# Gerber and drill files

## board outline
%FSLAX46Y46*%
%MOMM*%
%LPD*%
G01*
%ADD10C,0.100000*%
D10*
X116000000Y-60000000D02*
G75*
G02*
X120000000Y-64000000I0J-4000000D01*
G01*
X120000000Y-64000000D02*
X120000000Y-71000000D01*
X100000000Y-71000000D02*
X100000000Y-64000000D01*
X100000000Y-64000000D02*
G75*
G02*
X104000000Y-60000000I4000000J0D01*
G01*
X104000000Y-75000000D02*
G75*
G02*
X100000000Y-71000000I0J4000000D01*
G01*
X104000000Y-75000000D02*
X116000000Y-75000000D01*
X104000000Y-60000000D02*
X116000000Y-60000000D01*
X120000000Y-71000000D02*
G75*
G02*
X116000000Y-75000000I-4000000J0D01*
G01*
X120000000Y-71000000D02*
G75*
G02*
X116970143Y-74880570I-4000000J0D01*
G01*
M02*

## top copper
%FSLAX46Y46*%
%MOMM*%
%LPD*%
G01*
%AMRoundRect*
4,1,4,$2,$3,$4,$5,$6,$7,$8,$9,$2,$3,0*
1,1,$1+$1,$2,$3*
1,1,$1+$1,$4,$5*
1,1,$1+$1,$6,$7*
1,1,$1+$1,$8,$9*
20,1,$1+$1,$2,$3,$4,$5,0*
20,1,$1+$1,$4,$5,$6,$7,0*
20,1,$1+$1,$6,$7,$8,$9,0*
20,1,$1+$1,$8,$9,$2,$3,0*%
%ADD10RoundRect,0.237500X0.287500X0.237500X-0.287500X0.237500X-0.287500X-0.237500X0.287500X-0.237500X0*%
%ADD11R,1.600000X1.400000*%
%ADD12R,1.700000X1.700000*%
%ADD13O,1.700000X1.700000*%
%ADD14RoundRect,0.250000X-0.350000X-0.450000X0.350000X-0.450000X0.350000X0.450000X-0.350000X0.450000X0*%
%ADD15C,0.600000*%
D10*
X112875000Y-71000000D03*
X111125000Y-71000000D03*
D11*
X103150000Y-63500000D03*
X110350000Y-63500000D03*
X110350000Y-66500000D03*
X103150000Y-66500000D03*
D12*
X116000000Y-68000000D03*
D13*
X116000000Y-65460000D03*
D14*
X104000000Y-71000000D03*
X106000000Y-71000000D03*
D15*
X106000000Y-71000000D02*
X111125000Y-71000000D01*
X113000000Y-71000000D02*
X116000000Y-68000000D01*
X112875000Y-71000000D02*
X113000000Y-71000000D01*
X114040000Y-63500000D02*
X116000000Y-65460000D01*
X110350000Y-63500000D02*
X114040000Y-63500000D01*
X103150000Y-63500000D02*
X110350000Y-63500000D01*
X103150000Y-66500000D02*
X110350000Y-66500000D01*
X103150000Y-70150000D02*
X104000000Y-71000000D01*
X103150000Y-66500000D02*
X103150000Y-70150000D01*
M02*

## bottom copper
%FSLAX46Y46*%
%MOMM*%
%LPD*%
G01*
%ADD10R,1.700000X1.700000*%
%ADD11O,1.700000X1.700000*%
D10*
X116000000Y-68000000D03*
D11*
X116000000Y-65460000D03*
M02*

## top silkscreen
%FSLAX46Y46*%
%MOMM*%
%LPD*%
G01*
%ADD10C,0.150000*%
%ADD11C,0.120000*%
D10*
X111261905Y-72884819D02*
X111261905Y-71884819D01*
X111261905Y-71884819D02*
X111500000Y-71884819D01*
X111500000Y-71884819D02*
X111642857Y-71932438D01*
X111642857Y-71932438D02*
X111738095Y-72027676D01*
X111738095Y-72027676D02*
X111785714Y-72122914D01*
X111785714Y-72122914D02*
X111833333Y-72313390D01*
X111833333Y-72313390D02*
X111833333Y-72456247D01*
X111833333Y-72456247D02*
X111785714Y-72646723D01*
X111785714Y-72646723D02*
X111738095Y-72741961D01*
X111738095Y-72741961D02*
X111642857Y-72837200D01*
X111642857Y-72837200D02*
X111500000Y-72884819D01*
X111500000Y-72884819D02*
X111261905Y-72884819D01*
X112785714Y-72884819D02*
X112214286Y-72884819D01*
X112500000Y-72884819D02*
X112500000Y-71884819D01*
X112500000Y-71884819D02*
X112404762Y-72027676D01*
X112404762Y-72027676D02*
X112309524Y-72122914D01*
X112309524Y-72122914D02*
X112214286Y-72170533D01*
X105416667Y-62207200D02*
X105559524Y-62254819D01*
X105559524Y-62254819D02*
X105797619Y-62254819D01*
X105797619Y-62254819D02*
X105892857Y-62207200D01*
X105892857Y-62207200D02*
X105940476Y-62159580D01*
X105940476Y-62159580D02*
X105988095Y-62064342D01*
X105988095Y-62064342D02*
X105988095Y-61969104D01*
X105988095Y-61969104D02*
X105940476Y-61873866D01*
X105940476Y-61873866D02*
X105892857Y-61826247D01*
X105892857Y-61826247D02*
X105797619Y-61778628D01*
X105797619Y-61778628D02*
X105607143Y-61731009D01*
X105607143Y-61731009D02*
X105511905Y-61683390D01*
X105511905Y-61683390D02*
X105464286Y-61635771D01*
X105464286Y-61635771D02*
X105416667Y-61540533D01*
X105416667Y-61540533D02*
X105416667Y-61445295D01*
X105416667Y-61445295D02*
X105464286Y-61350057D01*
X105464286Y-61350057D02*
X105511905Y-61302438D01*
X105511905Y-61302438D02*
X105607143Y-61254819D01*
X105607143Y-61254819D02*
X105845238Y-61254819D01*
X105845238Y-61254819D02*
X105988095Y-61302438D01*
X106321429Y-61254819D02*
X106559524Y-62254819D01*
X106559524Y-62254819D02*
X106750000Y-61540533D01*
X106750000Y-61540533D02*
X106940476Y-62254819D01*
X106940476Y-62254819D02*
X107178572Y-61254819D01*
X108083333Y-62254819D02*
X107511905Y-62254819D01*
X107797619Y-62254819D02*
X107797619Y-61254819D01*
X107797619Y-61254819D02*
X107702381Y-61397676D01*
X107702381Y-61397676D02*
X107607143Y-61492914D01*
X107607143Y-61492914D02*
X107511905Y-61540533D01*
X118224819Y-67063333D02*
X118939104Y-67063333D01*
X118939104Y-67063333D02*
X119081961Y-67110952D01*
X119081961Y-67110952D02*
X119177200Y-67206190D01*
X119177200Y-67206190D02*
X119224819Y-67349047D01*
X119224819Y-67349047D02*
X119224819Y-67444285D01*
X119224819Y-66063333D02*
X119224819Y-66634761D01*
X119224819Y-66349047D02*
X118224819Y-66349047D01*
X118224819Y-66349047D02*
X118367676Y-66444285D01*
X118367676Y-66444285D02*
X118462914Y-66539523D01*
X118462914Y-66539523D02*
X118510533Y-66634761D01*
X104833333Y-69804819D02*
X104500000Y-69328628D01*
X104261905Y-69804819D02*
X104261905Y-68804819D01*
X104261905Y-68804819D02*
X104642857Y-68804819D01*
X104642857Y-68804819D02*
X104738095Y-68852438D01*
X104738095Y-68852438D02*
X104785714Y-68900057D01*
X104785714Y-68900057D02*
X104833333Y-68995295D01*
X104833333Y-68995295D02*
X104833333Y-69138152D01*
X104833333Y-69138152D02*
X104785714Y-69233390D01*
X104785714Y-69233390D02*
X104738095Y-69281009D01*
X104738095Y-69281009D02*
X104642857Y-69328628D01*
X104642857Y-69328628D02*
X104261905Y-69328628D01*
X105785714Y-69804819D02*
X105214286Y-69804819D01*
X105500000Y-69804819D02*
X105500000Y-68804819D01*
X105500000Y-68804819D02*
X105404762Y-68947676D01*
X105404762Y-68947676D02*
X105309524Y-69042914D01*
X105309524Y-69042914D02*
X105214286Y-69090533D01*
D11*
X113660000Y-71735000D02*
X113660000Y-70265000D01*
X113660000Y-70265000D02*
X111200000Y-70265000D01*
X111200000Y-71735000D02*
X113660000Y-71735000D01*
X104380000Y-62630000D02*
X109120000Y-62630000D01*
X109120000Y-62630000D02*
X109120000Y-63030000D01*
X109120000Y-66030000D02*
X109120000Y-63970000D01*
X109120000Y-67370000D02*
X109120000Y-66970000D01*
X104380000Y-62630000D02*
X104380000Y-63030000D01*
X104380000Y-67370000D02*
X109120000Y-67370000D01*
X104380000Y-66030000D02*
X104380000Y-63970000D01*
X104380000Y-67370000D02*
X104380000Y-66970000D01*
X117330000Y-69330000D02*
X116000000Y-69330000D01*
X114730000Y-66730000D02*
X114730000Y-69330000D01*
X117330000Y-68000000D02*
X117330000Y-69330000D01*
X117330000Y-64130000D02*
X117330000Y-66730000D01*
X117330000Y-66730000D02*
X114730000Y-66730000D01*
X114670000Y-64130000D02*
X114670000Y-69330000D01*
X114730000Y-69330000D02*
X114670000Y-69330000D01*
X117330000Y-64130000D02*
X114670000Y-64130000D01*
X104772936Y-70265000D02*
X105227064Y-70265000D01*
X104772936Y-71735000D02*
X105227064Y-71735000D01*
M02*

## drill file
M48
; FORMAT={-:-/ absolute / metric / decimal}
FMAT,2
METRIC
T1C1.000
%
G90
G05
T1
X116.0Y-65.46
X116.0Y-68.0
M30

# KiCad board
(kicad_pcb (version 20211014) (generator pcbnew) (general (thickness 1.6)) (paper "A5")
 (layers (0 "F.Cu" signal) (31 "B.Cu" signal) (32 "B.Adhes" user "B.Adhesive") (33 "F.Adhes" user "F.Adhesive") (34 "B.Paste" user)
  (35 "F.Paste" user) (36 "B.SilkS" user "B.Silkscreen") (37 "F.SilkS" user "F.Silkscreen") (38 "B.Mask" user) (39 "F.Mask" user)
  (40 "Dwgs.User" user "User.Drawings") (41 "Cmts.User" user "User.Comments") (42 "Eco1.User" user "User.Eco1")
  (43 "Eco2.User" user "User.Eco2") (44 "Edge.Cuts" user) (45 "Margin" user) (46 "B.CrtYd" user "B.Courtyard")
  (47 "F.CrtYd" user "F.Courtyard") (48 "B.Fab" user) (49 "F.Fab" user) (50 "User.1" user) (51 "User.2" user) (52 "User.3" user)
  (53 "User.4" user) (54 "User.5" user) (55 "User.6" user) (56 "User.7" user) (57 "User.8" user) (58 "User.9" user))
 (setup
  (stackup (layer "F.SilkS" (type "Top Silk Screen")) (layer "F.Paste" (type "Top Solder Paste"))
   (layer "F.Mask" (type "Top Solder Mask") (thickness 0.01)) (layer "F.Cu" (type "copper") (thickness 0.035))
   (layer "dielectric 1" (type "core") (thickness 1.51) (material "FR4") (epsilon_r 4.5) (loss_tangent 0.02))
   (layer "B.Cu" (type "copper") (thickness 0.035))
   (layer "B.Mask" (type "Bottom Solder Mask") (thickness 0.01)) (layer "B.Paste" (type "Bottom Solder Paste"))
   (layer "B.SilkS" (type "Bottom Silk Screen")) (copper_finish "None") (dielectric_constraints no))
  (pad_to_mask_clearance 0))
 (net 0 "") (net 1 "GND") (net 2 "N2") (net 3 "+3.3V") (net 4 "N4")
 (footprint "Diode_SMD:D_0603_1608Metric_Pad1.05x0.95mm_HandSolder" (layer "F.Cu") (at 112 71 180)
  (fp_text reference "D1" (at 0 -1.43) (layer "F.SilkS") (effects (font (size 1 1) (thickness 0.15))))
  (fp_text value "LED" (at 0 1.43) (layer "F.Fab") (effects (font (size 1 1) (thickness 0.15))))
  (fp_line (start -1.66 -0.735) (end -1.66 0.735) (layer "F.SilkS") (width 0.12))
  (fp_line (start -1.66 0.735) (end 0.8 0.735) (layer "F.SilkS") (width 0.12))
  (fp_line (start 0.8 -0.735) (end -1.66 -0.735) (layer "F.SilkS") (width 0.12))
  (pad "1" smd roundrect (at -0.875 0 180) (size 1.05 0.95) (layers "F.Cu" "F.Paste" "F.Mask") (roundrect_rratio 0.25) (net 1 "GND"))
  (pad "2" smd roundrect (at 0.875 0 180) (size 1.05 0.95) (layers "F.Cu" "F.Paste" "F.Mask") (roundrect_rratio 0.25) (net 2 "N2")))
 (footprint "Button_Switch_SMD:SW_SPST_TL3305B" (layer "F.Cu") (at 106.75 65)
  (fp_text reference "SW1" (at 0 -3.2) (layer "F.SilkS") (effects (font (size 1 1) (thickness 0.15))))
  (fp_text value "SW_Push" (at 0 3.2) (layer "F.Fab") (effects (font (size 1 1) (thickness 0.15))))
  (fp_line (start -2.37 -2.37) (end 2.37 -2.37) (layer "F.SilkS") (width 0.12))
  (fp_line (start 2.37 -2.37) (end 2.37 -1.97) (layer "F.SilkS") (width 0.12))
  (fp_line (start 2.37 1.03) (end 2.37 -1.03) (layer "F.SilkS") (width 0.12))
  (fp_line (start 2.37 2.37) (end 2.37 1.97) (layer "F.SilkS") (width 0.12))
  (fp_line (start -2.37 -2.37) (end -2.37 -1.97) (layer "F.SilkS") (width 0.12))
  (fp_line (start -2.37 2.37) (end 2.37 2.37) (layer "F.SilkS") (width 0.12))
  (fp_line (start -2.37 1.03) (end -2.37 -1.03) (layer "F.SilkS") (width 0.12))
  (fp_line (start -2.37 2.37) (end -2.37 1.97) (layer "F.SilkS") (width 0.12))
  (pad "1" smd rect (at -3.6 -1.5) (size 1.6 1.4) (layers "F.Cu" "F.Paste" "F.Mask") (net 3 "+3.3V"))
  (pad "1" smd rect (at 3.6 -1.5) (size 1.6 1.4) (layers "F.Cu" "F.Paste" "F.Mask") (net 3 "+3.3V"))
  (pad "2" smd rect (at 3.6 1.5) (size 1.6 1.4) (layers "F.Cu" "F.Paste" "F.Mask") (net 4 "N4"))
  (pad "2" smd rect (at -3.6 1.5) (size 1.6 1.4) (layers "F.Cu" "F.Paste" "F.Mask") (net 4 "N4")))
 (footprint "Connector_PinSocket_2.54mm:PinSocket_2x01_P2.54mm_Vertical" (layer "F.Cu") (at 116 68 -90)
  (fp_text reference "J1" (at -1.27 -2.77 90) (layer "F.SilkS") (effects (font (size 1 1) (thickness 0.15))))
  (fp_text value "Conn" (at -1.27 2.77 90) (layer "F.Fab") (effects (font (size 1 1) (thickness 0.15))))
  (fp_line (start 1.33 -1.33) (end 1.33 0) (layer "F.SilkS") (width 0.12))
  (fp_line (start -1.27 1.27) (end 1.33 1.27) (layer "F.SilkS") (width 0.12))
  (fp_line (start 0 -1.33) (end 1.33 -1.33) (layer "F.SilkS") (width 0.12))
  (fp_line (start -3.87 -1.33) (end -1.27 -1.33) (layer "F.SilkS") (width 0.12))
  (fp_line (start -1.27 -1.33) (end -1.27 1.27) (layer "F.SilkS") (width 0.12))
  (fp_line (start -3.87 1.33) (end 1.33 1.33) (layer "F.SilkS") (width 0.12))
  (fp_line (start 1.33 1.27) (end 1.33 1.33) (layer "F.SilkS") (width 0.12))
  (fp_line (start -3.87 -1.33) (end -3.87 1.33) (layer "F.SilkS") (width 0.12))
  (pad "1" thru_hole rect (at 0 0 270) (size 1.7 1.7) (drill 1) (layers *.Cu *.Mask) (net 1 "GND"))
  (pad "2" thru_hole oval (at -2.54 0 270) (size 1.7 1.7) (drill 1) (layers *.Cu *.Mask) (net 3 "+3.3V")))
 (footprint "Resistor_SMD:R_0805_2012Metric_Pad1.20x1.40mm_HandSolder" (layer "F.Cu") (at 105 71)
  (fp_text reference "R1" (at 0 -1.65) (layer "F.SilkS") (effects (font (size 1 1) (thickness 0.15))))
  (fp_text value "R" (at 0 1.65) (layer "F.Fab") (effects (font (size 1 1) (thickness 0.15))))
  (fp_line (start -0.227064 -0.735) (end 0.227064 -0.735) (layer "F.SilkS") (width 0.12))
  (fp_line (start -0.227064 0.735) (end 0.227064 0.735) (layer "F.SilkS") (width 0.12))
  (pad "1" smd roundrect (at -1 0) (size 1.2 1.4) (layers "F.Cu" "F.Paste" "F.Mask") (roundrect_rratio 0.208333) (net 4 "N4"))
  (pad "2" smd roundrect (at 1 0) (size 1.2 1.4) (layers "F.Cu" "F.Paste" "F.Mask") (roundrect_rratio 0.208333) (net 2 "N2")))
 (gr_arc (start 116 60) (mid 118.828427 61.171573) (end 120 64) (layer "Edge.Cuts") (width 0.1))
 (gr_line (start 120 64) (end 120 71) (layer "Edge.Cuts") (width 0.1))
 (gr_line (start 100 71) (end 100 64) (layer "Edge.Cuts") (width 0.1))
 (gr_arc (start 100 64) (mid 101.171573 61.171573) (end 104 60) (layer "Edge.Cuts") (width 0.1))
 (gr_arc (start 104 75) (mid 101.171573 73.828427) (end 100 71) (layer "Edge.Cuts") (width 0.1))
 (gr_line (start 104 75) (end 116 75) (layer "Edge.Cuts") (width 0.1))
 (gr_line (start 104 60) (end 116 60) (layer "Edge.Cuts") (width 0.1))
 (gr_arc (start 120 71) (mid 118.828427 73.828427) (end 116 75) (layer "Edge.Cuts") (width 0.1))
 (gr_arc (start 120 71) (mid 119.152822 73.461649) (end 116.970143 74.88057) (layer "Edge.Cuts") (width 0.1))
 (segment (start 106 71) (end 111.125 71) (width 0.6) (layer "F.Cu") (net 2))
 (segment (start 113 71) (end 116 68) (width 0.6) (layer "F.Cu") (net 1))
 (segment (start 112.875 71) (end 113 71) (width 0.6) (layer "F.Cu") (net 1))
 (segment (start 114.04 63.5) (end 116 65.46) (width 0.6) (layer "F.Cu") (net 3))
 (segment (start 110.35 63.5) (end 114.04 63.5) (width 0.6) (layer "F.Cu") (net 3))
 (segment (start 103.15 63.5) (end 110.35 63.5) (width 0.6) (layer "F.Cu") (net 3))
 (segment (start 103.15 66.5) (end 110.35 66.5) (width 0.6) (layer "F.Cu") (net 4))
 (segment (start 103.15 70.15) (end 104 71) (width 0.6) (layer "F.Cu") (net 4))
 (segment (start 103.15 66.5) (end 103.15 70.15) (width 0.6) (layer "F.Cu") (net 4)))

